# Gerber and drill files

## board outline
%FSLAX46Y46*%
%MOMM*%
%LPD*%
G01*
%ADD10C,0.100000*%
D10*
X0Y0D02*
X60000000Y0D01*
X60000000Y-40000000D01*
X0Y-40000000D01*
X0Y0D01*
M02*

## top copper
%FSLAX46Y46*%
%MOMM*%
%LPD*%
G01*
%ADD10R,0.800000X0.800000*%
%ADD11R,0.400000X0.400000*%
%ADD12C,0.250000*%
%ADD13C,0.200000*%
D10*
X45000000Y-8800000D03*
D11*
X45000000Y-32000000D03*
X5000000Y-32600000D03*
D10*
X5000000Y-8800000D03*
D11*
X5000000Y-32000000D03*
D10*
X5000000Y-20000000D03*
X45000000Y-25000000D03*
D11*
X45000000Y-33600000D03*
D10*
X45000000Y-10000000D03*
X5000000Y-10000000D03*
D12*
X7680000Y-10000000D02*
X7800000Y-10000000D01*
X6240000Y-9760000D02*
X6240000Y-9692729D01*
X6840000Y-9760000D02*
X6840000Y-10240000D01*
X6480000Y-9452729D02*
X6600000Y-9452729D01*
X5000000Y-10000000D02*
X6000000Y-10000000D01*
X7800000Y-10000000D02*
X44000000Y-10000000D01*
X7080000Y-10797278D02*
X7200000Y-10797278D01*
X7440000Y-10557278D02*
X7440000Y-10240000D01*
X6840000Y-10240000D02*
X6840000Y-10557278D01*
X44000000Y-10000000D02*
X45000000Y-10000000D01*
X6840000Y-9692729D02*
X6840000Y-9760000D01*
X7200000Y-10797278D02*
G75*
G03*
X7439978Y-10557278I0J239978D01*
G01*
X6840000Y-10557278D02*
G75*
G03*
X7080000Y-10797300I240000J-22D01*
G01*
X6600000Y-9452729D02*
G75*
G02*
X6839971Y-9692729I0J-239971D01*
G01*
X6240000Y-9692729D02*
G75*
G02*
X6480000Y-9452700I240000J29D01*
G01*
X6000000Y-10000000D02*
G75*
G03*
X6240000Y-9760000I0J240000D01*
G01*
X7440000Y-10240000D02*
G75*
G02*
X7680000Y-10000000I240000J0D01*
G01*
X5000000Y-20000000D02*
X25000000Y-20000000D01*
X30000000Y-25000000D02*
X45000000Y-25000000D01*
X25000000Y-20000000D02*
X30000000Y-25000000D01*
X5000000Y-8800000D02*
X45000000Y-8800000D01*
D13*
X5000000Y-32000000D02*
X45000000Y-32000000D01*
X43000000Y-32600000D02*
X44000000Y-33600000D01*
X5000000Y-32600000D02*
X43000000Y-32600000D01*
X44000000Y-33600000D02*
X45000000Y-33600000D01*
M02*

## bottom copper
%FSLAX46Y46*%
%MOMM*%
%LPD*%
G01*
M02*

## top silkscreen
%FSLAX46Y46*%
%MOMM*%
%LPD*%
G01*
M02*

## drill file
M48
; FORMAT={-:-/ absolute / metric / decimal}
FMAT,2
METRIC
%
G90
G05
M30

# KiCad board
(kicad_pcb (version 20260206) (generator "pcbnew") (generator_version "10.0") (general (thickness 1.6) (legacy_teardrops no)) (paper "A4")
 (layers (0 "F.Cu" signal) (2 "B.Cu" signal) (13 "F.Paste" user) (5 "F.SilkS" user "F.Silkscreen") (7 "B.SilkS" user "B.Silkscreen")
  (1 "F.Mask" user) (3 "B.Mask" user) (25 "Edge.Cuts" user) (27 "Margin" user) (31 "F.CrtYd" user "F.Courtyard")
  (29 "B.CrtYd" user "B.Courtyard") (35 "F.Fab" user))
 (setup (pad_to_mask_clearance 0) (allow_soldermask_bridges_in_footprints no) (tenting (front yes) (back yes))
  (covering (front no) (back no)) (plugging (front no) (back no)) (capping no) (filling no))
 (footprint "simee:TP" (layer "F.Cu") (at 45 8.8)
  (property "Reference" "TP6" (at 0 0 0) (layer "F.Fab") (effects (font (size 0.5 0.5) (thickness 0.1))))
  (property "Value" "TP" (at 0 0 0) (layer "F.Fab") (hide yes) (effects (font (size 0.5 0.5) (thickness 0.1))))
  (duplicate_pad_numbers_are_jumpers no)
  (pad "1" smd rect (at 0 0) (size 0.8 0.8) (layers "F.Cu" "F.Mask") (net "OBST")))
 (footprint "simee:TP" (layer "F.Cu") (at 45 32)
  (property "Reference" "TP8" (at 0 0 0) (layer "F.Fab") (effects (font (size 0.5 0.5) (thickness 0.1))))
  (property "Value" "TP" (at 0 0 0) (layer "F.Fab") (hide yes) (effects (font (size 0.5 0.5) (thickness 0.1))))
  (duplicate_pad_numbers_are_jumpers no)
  (pad "1" smd rect (at 0 0) (size 0.4 0.4) (layers "F.Cu" "F.Mask") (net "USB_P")))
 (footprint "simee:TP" (layer "F.Cu") (at 5 32.6)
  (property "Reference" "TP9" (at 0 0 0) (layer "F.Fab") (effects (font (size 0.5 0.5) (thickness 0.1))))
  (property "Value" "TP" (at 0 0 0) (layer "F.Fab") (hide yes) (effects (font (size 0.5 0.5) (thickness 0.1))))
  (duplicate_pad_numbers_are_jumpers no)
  (pad "1" smd rect (at 0 0) (size 0.4 0.4) (layers "F.Cu" "F.Mask") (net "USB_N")))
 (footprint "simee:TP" (layer "F.Cu") (at 5 8.8)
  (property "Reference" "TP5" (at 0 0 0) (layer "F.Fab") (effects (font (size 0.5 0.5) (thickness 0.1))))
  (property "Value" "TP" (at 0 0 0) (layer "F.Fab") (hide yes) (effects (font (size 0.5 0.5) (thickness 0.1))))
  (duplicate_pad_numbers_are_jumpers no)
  (pad "1" smd rect (at 0 0) (size 0.8 0.8) (layers "F.Cu" "F.Mask") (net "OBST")))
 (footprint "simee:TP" (layer "F.Cu") (at 5 32)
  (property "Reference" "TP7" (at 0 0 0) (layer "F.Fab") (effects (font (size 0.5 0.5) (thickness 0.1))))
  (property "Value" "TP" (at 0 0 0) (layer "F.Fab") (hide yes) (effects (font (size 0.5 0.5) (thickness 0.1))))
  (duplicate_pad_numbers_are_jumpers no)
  (pad "1" smd rect (at 0 0) (size 0.4 0.4) (layers "F.Cu" "F.Mask") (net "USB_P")))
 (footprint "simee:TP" (layer "F.Cu") (at 5 20)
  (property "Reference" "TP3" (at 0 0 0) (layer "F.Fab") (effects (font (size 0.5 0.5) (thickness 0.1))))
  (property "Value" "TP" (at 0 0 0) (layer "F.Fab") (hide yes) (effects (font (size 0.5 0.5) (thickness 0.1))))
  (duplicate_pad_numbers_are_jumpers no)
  (pad "1" smd rect (at 0 0) (size 0.8 0.8) (layers "F.Cu" "F.Mask") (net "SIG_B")))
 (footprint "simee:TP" (layer "F.Cu") (at 45 25)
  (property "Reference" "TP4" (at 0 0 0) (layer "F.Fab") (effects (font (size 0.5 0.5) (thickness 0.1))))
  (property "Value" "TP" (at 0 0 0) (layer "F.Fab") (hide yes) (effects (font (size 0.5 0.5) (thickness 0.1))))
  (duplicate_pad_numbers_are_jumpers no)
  (pad "1" smd rect (at 0 0) (size 0.8 0.8) (layers "F.Cu" "F.Mask") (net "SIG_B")))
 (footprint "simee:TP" (layer "F.Cu") (at 45 33.6)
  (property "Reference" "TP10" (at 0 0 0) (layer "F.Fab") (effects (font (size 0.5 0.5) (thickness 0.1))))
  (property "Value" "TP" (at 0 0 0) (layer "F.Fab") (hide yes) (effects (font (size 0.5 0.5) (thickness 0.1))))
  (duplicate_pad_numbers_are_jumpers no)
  (pad "1" smd rect (at 0 0) (size 0.4 0.4) (layers "F.Cu" "F.Mask") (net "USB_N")))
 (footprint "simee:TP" (layer "F.Cu") (at 45 10)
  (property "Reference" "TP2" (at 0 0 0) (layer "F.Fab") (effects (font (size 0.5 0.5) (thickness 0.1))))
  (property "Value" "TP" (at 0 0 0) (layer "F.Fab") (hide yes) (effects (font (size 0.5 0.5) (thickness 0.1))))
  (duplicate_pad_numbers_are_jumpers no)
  (pad "1" smd rect (at 0 0) (size 0.8 0.8) (layers "F.Cu" "F.Mask") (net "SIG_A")))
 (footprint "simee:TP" (layer "F.Cu") (at 5 10)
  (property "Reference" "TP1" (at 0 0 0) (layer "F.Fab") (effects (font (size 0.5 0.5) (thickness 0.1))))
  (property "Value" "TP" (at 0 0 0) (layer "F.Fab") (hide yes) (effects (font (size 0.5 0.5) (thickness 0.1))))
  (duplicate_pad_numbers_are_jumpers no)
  (pad "1" smd rect (at 0 0) (size 0.8 0.8) (layers "F.Cu" "F.Mask") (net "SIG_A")))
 (gr_rect (start 0 0) (end 60 40) (stroke (width 0.1) (type default)) (fill no) (layer "Edge.Cuts"))
 (segment (start 7.68 10) (end 7.8 10) (width 0.25) (layer "F.Cu") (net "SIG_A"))
 (segment (start 6.24 9.76) (end 6.24 9.692729) (width 0.25) (layer "F.Cu") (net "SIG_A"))
 (segment (start 6.84 9.76) (end 6.84 10.24) (width 0.25) (layer "F.Cu") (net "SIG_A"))
 (segment (start 6.48 9.452729) (end 6.6 9.452729) (width 0.25) (layer "F.Cu") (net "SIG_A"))
 (segment (start 5 10) (end 6 10) (width 0.25) (layer "F.Cu") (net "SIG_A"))
 (segment (start 7.8 10) (end 44 10) (width 0.25) (layer "F.Cu") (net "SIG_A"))
 (segment (start 7.08 10.797278) (end 7.2 10.797278) (width 0.25) (layer "F.Cu") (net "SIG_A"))
 (segment (start 7.44 10.557278) (end 7.44 10.24) (width 0.25) (layer "F.Cu") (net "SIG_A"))
 (segment (start 6.84 10.24) (end 6.84 10.557278) (width 0.25) (layer "F.Cu") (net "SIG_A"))
 (segment (start 44 10) (end 45 10) (width 0.25) (layer "F.Cu") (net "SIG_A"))
 (segment (start 6.84 9.692729) (end 6.84 9.76) (width 0.25) (layer "F.Cu") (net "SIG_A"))
 (arc (start 7.2 10.797278) (mid 7.369706 10.726984) (end 7.44 10.557278) (width 0.25) (layer "F.Cu") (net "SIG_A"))
 (arc (start 6.84 10.557278) (mid 6.910294 10.726984) (end 7.08 10.797278) (width 0.25) (layer "F.Cu") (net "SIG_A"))
 (arc (start 6.6 9.452729) (mid 6.769706 9.523023) (end 6.84 9.692729) (width 0.25) (layer "F.Cu") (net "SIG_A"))
 (arc (start 6.24 9.692729) (mid 6.310294 9.523023) (end 6.48 9.452729) (width 0.25) (layer "F.Cu") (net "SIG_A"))
 (arc (start 6 10) (mid 6.169706 9.929706) (end 6.24 9.76) (width 0.25) (layer "F.Cu") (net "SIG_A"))
 (arc (start 7.44 10.24) (mid 7.510294 10.070294) (end 7.68 10) (width 0.25) (layer "F.Cu") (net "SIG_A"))
 (segment (start 5 20) (end 25 20) (width 0.25) (layer "F.Cu") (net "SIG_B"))
 (segment (start 30 25) (end 45 25) (width 0.25) (layer "F.Cu") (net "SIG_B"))
 (segment (start 25 20) (end 30 25) (width 0.25) (layer "F.Cu") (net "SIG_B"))
 (segment (start 5 8.8) (end 45 8.8) (width 0.25) (layer "F.Cu") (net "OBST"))
 (segment (start 5 32) (end 45 32) (width 0.2) (layer "F.Cu") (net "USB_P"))
 (segment (start 43 32.6) (end 44 33.6) (width 0.2) (layer "F.Cu") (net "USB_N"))
 (segment (start 5 32.6) (end 43 32.6) (width 0.2) (layer "F.Cu") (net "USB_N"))
 (segment (start 44 33.6) (end 45 33.6) (width 0.2) (layer "F.Cu") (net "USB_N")))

